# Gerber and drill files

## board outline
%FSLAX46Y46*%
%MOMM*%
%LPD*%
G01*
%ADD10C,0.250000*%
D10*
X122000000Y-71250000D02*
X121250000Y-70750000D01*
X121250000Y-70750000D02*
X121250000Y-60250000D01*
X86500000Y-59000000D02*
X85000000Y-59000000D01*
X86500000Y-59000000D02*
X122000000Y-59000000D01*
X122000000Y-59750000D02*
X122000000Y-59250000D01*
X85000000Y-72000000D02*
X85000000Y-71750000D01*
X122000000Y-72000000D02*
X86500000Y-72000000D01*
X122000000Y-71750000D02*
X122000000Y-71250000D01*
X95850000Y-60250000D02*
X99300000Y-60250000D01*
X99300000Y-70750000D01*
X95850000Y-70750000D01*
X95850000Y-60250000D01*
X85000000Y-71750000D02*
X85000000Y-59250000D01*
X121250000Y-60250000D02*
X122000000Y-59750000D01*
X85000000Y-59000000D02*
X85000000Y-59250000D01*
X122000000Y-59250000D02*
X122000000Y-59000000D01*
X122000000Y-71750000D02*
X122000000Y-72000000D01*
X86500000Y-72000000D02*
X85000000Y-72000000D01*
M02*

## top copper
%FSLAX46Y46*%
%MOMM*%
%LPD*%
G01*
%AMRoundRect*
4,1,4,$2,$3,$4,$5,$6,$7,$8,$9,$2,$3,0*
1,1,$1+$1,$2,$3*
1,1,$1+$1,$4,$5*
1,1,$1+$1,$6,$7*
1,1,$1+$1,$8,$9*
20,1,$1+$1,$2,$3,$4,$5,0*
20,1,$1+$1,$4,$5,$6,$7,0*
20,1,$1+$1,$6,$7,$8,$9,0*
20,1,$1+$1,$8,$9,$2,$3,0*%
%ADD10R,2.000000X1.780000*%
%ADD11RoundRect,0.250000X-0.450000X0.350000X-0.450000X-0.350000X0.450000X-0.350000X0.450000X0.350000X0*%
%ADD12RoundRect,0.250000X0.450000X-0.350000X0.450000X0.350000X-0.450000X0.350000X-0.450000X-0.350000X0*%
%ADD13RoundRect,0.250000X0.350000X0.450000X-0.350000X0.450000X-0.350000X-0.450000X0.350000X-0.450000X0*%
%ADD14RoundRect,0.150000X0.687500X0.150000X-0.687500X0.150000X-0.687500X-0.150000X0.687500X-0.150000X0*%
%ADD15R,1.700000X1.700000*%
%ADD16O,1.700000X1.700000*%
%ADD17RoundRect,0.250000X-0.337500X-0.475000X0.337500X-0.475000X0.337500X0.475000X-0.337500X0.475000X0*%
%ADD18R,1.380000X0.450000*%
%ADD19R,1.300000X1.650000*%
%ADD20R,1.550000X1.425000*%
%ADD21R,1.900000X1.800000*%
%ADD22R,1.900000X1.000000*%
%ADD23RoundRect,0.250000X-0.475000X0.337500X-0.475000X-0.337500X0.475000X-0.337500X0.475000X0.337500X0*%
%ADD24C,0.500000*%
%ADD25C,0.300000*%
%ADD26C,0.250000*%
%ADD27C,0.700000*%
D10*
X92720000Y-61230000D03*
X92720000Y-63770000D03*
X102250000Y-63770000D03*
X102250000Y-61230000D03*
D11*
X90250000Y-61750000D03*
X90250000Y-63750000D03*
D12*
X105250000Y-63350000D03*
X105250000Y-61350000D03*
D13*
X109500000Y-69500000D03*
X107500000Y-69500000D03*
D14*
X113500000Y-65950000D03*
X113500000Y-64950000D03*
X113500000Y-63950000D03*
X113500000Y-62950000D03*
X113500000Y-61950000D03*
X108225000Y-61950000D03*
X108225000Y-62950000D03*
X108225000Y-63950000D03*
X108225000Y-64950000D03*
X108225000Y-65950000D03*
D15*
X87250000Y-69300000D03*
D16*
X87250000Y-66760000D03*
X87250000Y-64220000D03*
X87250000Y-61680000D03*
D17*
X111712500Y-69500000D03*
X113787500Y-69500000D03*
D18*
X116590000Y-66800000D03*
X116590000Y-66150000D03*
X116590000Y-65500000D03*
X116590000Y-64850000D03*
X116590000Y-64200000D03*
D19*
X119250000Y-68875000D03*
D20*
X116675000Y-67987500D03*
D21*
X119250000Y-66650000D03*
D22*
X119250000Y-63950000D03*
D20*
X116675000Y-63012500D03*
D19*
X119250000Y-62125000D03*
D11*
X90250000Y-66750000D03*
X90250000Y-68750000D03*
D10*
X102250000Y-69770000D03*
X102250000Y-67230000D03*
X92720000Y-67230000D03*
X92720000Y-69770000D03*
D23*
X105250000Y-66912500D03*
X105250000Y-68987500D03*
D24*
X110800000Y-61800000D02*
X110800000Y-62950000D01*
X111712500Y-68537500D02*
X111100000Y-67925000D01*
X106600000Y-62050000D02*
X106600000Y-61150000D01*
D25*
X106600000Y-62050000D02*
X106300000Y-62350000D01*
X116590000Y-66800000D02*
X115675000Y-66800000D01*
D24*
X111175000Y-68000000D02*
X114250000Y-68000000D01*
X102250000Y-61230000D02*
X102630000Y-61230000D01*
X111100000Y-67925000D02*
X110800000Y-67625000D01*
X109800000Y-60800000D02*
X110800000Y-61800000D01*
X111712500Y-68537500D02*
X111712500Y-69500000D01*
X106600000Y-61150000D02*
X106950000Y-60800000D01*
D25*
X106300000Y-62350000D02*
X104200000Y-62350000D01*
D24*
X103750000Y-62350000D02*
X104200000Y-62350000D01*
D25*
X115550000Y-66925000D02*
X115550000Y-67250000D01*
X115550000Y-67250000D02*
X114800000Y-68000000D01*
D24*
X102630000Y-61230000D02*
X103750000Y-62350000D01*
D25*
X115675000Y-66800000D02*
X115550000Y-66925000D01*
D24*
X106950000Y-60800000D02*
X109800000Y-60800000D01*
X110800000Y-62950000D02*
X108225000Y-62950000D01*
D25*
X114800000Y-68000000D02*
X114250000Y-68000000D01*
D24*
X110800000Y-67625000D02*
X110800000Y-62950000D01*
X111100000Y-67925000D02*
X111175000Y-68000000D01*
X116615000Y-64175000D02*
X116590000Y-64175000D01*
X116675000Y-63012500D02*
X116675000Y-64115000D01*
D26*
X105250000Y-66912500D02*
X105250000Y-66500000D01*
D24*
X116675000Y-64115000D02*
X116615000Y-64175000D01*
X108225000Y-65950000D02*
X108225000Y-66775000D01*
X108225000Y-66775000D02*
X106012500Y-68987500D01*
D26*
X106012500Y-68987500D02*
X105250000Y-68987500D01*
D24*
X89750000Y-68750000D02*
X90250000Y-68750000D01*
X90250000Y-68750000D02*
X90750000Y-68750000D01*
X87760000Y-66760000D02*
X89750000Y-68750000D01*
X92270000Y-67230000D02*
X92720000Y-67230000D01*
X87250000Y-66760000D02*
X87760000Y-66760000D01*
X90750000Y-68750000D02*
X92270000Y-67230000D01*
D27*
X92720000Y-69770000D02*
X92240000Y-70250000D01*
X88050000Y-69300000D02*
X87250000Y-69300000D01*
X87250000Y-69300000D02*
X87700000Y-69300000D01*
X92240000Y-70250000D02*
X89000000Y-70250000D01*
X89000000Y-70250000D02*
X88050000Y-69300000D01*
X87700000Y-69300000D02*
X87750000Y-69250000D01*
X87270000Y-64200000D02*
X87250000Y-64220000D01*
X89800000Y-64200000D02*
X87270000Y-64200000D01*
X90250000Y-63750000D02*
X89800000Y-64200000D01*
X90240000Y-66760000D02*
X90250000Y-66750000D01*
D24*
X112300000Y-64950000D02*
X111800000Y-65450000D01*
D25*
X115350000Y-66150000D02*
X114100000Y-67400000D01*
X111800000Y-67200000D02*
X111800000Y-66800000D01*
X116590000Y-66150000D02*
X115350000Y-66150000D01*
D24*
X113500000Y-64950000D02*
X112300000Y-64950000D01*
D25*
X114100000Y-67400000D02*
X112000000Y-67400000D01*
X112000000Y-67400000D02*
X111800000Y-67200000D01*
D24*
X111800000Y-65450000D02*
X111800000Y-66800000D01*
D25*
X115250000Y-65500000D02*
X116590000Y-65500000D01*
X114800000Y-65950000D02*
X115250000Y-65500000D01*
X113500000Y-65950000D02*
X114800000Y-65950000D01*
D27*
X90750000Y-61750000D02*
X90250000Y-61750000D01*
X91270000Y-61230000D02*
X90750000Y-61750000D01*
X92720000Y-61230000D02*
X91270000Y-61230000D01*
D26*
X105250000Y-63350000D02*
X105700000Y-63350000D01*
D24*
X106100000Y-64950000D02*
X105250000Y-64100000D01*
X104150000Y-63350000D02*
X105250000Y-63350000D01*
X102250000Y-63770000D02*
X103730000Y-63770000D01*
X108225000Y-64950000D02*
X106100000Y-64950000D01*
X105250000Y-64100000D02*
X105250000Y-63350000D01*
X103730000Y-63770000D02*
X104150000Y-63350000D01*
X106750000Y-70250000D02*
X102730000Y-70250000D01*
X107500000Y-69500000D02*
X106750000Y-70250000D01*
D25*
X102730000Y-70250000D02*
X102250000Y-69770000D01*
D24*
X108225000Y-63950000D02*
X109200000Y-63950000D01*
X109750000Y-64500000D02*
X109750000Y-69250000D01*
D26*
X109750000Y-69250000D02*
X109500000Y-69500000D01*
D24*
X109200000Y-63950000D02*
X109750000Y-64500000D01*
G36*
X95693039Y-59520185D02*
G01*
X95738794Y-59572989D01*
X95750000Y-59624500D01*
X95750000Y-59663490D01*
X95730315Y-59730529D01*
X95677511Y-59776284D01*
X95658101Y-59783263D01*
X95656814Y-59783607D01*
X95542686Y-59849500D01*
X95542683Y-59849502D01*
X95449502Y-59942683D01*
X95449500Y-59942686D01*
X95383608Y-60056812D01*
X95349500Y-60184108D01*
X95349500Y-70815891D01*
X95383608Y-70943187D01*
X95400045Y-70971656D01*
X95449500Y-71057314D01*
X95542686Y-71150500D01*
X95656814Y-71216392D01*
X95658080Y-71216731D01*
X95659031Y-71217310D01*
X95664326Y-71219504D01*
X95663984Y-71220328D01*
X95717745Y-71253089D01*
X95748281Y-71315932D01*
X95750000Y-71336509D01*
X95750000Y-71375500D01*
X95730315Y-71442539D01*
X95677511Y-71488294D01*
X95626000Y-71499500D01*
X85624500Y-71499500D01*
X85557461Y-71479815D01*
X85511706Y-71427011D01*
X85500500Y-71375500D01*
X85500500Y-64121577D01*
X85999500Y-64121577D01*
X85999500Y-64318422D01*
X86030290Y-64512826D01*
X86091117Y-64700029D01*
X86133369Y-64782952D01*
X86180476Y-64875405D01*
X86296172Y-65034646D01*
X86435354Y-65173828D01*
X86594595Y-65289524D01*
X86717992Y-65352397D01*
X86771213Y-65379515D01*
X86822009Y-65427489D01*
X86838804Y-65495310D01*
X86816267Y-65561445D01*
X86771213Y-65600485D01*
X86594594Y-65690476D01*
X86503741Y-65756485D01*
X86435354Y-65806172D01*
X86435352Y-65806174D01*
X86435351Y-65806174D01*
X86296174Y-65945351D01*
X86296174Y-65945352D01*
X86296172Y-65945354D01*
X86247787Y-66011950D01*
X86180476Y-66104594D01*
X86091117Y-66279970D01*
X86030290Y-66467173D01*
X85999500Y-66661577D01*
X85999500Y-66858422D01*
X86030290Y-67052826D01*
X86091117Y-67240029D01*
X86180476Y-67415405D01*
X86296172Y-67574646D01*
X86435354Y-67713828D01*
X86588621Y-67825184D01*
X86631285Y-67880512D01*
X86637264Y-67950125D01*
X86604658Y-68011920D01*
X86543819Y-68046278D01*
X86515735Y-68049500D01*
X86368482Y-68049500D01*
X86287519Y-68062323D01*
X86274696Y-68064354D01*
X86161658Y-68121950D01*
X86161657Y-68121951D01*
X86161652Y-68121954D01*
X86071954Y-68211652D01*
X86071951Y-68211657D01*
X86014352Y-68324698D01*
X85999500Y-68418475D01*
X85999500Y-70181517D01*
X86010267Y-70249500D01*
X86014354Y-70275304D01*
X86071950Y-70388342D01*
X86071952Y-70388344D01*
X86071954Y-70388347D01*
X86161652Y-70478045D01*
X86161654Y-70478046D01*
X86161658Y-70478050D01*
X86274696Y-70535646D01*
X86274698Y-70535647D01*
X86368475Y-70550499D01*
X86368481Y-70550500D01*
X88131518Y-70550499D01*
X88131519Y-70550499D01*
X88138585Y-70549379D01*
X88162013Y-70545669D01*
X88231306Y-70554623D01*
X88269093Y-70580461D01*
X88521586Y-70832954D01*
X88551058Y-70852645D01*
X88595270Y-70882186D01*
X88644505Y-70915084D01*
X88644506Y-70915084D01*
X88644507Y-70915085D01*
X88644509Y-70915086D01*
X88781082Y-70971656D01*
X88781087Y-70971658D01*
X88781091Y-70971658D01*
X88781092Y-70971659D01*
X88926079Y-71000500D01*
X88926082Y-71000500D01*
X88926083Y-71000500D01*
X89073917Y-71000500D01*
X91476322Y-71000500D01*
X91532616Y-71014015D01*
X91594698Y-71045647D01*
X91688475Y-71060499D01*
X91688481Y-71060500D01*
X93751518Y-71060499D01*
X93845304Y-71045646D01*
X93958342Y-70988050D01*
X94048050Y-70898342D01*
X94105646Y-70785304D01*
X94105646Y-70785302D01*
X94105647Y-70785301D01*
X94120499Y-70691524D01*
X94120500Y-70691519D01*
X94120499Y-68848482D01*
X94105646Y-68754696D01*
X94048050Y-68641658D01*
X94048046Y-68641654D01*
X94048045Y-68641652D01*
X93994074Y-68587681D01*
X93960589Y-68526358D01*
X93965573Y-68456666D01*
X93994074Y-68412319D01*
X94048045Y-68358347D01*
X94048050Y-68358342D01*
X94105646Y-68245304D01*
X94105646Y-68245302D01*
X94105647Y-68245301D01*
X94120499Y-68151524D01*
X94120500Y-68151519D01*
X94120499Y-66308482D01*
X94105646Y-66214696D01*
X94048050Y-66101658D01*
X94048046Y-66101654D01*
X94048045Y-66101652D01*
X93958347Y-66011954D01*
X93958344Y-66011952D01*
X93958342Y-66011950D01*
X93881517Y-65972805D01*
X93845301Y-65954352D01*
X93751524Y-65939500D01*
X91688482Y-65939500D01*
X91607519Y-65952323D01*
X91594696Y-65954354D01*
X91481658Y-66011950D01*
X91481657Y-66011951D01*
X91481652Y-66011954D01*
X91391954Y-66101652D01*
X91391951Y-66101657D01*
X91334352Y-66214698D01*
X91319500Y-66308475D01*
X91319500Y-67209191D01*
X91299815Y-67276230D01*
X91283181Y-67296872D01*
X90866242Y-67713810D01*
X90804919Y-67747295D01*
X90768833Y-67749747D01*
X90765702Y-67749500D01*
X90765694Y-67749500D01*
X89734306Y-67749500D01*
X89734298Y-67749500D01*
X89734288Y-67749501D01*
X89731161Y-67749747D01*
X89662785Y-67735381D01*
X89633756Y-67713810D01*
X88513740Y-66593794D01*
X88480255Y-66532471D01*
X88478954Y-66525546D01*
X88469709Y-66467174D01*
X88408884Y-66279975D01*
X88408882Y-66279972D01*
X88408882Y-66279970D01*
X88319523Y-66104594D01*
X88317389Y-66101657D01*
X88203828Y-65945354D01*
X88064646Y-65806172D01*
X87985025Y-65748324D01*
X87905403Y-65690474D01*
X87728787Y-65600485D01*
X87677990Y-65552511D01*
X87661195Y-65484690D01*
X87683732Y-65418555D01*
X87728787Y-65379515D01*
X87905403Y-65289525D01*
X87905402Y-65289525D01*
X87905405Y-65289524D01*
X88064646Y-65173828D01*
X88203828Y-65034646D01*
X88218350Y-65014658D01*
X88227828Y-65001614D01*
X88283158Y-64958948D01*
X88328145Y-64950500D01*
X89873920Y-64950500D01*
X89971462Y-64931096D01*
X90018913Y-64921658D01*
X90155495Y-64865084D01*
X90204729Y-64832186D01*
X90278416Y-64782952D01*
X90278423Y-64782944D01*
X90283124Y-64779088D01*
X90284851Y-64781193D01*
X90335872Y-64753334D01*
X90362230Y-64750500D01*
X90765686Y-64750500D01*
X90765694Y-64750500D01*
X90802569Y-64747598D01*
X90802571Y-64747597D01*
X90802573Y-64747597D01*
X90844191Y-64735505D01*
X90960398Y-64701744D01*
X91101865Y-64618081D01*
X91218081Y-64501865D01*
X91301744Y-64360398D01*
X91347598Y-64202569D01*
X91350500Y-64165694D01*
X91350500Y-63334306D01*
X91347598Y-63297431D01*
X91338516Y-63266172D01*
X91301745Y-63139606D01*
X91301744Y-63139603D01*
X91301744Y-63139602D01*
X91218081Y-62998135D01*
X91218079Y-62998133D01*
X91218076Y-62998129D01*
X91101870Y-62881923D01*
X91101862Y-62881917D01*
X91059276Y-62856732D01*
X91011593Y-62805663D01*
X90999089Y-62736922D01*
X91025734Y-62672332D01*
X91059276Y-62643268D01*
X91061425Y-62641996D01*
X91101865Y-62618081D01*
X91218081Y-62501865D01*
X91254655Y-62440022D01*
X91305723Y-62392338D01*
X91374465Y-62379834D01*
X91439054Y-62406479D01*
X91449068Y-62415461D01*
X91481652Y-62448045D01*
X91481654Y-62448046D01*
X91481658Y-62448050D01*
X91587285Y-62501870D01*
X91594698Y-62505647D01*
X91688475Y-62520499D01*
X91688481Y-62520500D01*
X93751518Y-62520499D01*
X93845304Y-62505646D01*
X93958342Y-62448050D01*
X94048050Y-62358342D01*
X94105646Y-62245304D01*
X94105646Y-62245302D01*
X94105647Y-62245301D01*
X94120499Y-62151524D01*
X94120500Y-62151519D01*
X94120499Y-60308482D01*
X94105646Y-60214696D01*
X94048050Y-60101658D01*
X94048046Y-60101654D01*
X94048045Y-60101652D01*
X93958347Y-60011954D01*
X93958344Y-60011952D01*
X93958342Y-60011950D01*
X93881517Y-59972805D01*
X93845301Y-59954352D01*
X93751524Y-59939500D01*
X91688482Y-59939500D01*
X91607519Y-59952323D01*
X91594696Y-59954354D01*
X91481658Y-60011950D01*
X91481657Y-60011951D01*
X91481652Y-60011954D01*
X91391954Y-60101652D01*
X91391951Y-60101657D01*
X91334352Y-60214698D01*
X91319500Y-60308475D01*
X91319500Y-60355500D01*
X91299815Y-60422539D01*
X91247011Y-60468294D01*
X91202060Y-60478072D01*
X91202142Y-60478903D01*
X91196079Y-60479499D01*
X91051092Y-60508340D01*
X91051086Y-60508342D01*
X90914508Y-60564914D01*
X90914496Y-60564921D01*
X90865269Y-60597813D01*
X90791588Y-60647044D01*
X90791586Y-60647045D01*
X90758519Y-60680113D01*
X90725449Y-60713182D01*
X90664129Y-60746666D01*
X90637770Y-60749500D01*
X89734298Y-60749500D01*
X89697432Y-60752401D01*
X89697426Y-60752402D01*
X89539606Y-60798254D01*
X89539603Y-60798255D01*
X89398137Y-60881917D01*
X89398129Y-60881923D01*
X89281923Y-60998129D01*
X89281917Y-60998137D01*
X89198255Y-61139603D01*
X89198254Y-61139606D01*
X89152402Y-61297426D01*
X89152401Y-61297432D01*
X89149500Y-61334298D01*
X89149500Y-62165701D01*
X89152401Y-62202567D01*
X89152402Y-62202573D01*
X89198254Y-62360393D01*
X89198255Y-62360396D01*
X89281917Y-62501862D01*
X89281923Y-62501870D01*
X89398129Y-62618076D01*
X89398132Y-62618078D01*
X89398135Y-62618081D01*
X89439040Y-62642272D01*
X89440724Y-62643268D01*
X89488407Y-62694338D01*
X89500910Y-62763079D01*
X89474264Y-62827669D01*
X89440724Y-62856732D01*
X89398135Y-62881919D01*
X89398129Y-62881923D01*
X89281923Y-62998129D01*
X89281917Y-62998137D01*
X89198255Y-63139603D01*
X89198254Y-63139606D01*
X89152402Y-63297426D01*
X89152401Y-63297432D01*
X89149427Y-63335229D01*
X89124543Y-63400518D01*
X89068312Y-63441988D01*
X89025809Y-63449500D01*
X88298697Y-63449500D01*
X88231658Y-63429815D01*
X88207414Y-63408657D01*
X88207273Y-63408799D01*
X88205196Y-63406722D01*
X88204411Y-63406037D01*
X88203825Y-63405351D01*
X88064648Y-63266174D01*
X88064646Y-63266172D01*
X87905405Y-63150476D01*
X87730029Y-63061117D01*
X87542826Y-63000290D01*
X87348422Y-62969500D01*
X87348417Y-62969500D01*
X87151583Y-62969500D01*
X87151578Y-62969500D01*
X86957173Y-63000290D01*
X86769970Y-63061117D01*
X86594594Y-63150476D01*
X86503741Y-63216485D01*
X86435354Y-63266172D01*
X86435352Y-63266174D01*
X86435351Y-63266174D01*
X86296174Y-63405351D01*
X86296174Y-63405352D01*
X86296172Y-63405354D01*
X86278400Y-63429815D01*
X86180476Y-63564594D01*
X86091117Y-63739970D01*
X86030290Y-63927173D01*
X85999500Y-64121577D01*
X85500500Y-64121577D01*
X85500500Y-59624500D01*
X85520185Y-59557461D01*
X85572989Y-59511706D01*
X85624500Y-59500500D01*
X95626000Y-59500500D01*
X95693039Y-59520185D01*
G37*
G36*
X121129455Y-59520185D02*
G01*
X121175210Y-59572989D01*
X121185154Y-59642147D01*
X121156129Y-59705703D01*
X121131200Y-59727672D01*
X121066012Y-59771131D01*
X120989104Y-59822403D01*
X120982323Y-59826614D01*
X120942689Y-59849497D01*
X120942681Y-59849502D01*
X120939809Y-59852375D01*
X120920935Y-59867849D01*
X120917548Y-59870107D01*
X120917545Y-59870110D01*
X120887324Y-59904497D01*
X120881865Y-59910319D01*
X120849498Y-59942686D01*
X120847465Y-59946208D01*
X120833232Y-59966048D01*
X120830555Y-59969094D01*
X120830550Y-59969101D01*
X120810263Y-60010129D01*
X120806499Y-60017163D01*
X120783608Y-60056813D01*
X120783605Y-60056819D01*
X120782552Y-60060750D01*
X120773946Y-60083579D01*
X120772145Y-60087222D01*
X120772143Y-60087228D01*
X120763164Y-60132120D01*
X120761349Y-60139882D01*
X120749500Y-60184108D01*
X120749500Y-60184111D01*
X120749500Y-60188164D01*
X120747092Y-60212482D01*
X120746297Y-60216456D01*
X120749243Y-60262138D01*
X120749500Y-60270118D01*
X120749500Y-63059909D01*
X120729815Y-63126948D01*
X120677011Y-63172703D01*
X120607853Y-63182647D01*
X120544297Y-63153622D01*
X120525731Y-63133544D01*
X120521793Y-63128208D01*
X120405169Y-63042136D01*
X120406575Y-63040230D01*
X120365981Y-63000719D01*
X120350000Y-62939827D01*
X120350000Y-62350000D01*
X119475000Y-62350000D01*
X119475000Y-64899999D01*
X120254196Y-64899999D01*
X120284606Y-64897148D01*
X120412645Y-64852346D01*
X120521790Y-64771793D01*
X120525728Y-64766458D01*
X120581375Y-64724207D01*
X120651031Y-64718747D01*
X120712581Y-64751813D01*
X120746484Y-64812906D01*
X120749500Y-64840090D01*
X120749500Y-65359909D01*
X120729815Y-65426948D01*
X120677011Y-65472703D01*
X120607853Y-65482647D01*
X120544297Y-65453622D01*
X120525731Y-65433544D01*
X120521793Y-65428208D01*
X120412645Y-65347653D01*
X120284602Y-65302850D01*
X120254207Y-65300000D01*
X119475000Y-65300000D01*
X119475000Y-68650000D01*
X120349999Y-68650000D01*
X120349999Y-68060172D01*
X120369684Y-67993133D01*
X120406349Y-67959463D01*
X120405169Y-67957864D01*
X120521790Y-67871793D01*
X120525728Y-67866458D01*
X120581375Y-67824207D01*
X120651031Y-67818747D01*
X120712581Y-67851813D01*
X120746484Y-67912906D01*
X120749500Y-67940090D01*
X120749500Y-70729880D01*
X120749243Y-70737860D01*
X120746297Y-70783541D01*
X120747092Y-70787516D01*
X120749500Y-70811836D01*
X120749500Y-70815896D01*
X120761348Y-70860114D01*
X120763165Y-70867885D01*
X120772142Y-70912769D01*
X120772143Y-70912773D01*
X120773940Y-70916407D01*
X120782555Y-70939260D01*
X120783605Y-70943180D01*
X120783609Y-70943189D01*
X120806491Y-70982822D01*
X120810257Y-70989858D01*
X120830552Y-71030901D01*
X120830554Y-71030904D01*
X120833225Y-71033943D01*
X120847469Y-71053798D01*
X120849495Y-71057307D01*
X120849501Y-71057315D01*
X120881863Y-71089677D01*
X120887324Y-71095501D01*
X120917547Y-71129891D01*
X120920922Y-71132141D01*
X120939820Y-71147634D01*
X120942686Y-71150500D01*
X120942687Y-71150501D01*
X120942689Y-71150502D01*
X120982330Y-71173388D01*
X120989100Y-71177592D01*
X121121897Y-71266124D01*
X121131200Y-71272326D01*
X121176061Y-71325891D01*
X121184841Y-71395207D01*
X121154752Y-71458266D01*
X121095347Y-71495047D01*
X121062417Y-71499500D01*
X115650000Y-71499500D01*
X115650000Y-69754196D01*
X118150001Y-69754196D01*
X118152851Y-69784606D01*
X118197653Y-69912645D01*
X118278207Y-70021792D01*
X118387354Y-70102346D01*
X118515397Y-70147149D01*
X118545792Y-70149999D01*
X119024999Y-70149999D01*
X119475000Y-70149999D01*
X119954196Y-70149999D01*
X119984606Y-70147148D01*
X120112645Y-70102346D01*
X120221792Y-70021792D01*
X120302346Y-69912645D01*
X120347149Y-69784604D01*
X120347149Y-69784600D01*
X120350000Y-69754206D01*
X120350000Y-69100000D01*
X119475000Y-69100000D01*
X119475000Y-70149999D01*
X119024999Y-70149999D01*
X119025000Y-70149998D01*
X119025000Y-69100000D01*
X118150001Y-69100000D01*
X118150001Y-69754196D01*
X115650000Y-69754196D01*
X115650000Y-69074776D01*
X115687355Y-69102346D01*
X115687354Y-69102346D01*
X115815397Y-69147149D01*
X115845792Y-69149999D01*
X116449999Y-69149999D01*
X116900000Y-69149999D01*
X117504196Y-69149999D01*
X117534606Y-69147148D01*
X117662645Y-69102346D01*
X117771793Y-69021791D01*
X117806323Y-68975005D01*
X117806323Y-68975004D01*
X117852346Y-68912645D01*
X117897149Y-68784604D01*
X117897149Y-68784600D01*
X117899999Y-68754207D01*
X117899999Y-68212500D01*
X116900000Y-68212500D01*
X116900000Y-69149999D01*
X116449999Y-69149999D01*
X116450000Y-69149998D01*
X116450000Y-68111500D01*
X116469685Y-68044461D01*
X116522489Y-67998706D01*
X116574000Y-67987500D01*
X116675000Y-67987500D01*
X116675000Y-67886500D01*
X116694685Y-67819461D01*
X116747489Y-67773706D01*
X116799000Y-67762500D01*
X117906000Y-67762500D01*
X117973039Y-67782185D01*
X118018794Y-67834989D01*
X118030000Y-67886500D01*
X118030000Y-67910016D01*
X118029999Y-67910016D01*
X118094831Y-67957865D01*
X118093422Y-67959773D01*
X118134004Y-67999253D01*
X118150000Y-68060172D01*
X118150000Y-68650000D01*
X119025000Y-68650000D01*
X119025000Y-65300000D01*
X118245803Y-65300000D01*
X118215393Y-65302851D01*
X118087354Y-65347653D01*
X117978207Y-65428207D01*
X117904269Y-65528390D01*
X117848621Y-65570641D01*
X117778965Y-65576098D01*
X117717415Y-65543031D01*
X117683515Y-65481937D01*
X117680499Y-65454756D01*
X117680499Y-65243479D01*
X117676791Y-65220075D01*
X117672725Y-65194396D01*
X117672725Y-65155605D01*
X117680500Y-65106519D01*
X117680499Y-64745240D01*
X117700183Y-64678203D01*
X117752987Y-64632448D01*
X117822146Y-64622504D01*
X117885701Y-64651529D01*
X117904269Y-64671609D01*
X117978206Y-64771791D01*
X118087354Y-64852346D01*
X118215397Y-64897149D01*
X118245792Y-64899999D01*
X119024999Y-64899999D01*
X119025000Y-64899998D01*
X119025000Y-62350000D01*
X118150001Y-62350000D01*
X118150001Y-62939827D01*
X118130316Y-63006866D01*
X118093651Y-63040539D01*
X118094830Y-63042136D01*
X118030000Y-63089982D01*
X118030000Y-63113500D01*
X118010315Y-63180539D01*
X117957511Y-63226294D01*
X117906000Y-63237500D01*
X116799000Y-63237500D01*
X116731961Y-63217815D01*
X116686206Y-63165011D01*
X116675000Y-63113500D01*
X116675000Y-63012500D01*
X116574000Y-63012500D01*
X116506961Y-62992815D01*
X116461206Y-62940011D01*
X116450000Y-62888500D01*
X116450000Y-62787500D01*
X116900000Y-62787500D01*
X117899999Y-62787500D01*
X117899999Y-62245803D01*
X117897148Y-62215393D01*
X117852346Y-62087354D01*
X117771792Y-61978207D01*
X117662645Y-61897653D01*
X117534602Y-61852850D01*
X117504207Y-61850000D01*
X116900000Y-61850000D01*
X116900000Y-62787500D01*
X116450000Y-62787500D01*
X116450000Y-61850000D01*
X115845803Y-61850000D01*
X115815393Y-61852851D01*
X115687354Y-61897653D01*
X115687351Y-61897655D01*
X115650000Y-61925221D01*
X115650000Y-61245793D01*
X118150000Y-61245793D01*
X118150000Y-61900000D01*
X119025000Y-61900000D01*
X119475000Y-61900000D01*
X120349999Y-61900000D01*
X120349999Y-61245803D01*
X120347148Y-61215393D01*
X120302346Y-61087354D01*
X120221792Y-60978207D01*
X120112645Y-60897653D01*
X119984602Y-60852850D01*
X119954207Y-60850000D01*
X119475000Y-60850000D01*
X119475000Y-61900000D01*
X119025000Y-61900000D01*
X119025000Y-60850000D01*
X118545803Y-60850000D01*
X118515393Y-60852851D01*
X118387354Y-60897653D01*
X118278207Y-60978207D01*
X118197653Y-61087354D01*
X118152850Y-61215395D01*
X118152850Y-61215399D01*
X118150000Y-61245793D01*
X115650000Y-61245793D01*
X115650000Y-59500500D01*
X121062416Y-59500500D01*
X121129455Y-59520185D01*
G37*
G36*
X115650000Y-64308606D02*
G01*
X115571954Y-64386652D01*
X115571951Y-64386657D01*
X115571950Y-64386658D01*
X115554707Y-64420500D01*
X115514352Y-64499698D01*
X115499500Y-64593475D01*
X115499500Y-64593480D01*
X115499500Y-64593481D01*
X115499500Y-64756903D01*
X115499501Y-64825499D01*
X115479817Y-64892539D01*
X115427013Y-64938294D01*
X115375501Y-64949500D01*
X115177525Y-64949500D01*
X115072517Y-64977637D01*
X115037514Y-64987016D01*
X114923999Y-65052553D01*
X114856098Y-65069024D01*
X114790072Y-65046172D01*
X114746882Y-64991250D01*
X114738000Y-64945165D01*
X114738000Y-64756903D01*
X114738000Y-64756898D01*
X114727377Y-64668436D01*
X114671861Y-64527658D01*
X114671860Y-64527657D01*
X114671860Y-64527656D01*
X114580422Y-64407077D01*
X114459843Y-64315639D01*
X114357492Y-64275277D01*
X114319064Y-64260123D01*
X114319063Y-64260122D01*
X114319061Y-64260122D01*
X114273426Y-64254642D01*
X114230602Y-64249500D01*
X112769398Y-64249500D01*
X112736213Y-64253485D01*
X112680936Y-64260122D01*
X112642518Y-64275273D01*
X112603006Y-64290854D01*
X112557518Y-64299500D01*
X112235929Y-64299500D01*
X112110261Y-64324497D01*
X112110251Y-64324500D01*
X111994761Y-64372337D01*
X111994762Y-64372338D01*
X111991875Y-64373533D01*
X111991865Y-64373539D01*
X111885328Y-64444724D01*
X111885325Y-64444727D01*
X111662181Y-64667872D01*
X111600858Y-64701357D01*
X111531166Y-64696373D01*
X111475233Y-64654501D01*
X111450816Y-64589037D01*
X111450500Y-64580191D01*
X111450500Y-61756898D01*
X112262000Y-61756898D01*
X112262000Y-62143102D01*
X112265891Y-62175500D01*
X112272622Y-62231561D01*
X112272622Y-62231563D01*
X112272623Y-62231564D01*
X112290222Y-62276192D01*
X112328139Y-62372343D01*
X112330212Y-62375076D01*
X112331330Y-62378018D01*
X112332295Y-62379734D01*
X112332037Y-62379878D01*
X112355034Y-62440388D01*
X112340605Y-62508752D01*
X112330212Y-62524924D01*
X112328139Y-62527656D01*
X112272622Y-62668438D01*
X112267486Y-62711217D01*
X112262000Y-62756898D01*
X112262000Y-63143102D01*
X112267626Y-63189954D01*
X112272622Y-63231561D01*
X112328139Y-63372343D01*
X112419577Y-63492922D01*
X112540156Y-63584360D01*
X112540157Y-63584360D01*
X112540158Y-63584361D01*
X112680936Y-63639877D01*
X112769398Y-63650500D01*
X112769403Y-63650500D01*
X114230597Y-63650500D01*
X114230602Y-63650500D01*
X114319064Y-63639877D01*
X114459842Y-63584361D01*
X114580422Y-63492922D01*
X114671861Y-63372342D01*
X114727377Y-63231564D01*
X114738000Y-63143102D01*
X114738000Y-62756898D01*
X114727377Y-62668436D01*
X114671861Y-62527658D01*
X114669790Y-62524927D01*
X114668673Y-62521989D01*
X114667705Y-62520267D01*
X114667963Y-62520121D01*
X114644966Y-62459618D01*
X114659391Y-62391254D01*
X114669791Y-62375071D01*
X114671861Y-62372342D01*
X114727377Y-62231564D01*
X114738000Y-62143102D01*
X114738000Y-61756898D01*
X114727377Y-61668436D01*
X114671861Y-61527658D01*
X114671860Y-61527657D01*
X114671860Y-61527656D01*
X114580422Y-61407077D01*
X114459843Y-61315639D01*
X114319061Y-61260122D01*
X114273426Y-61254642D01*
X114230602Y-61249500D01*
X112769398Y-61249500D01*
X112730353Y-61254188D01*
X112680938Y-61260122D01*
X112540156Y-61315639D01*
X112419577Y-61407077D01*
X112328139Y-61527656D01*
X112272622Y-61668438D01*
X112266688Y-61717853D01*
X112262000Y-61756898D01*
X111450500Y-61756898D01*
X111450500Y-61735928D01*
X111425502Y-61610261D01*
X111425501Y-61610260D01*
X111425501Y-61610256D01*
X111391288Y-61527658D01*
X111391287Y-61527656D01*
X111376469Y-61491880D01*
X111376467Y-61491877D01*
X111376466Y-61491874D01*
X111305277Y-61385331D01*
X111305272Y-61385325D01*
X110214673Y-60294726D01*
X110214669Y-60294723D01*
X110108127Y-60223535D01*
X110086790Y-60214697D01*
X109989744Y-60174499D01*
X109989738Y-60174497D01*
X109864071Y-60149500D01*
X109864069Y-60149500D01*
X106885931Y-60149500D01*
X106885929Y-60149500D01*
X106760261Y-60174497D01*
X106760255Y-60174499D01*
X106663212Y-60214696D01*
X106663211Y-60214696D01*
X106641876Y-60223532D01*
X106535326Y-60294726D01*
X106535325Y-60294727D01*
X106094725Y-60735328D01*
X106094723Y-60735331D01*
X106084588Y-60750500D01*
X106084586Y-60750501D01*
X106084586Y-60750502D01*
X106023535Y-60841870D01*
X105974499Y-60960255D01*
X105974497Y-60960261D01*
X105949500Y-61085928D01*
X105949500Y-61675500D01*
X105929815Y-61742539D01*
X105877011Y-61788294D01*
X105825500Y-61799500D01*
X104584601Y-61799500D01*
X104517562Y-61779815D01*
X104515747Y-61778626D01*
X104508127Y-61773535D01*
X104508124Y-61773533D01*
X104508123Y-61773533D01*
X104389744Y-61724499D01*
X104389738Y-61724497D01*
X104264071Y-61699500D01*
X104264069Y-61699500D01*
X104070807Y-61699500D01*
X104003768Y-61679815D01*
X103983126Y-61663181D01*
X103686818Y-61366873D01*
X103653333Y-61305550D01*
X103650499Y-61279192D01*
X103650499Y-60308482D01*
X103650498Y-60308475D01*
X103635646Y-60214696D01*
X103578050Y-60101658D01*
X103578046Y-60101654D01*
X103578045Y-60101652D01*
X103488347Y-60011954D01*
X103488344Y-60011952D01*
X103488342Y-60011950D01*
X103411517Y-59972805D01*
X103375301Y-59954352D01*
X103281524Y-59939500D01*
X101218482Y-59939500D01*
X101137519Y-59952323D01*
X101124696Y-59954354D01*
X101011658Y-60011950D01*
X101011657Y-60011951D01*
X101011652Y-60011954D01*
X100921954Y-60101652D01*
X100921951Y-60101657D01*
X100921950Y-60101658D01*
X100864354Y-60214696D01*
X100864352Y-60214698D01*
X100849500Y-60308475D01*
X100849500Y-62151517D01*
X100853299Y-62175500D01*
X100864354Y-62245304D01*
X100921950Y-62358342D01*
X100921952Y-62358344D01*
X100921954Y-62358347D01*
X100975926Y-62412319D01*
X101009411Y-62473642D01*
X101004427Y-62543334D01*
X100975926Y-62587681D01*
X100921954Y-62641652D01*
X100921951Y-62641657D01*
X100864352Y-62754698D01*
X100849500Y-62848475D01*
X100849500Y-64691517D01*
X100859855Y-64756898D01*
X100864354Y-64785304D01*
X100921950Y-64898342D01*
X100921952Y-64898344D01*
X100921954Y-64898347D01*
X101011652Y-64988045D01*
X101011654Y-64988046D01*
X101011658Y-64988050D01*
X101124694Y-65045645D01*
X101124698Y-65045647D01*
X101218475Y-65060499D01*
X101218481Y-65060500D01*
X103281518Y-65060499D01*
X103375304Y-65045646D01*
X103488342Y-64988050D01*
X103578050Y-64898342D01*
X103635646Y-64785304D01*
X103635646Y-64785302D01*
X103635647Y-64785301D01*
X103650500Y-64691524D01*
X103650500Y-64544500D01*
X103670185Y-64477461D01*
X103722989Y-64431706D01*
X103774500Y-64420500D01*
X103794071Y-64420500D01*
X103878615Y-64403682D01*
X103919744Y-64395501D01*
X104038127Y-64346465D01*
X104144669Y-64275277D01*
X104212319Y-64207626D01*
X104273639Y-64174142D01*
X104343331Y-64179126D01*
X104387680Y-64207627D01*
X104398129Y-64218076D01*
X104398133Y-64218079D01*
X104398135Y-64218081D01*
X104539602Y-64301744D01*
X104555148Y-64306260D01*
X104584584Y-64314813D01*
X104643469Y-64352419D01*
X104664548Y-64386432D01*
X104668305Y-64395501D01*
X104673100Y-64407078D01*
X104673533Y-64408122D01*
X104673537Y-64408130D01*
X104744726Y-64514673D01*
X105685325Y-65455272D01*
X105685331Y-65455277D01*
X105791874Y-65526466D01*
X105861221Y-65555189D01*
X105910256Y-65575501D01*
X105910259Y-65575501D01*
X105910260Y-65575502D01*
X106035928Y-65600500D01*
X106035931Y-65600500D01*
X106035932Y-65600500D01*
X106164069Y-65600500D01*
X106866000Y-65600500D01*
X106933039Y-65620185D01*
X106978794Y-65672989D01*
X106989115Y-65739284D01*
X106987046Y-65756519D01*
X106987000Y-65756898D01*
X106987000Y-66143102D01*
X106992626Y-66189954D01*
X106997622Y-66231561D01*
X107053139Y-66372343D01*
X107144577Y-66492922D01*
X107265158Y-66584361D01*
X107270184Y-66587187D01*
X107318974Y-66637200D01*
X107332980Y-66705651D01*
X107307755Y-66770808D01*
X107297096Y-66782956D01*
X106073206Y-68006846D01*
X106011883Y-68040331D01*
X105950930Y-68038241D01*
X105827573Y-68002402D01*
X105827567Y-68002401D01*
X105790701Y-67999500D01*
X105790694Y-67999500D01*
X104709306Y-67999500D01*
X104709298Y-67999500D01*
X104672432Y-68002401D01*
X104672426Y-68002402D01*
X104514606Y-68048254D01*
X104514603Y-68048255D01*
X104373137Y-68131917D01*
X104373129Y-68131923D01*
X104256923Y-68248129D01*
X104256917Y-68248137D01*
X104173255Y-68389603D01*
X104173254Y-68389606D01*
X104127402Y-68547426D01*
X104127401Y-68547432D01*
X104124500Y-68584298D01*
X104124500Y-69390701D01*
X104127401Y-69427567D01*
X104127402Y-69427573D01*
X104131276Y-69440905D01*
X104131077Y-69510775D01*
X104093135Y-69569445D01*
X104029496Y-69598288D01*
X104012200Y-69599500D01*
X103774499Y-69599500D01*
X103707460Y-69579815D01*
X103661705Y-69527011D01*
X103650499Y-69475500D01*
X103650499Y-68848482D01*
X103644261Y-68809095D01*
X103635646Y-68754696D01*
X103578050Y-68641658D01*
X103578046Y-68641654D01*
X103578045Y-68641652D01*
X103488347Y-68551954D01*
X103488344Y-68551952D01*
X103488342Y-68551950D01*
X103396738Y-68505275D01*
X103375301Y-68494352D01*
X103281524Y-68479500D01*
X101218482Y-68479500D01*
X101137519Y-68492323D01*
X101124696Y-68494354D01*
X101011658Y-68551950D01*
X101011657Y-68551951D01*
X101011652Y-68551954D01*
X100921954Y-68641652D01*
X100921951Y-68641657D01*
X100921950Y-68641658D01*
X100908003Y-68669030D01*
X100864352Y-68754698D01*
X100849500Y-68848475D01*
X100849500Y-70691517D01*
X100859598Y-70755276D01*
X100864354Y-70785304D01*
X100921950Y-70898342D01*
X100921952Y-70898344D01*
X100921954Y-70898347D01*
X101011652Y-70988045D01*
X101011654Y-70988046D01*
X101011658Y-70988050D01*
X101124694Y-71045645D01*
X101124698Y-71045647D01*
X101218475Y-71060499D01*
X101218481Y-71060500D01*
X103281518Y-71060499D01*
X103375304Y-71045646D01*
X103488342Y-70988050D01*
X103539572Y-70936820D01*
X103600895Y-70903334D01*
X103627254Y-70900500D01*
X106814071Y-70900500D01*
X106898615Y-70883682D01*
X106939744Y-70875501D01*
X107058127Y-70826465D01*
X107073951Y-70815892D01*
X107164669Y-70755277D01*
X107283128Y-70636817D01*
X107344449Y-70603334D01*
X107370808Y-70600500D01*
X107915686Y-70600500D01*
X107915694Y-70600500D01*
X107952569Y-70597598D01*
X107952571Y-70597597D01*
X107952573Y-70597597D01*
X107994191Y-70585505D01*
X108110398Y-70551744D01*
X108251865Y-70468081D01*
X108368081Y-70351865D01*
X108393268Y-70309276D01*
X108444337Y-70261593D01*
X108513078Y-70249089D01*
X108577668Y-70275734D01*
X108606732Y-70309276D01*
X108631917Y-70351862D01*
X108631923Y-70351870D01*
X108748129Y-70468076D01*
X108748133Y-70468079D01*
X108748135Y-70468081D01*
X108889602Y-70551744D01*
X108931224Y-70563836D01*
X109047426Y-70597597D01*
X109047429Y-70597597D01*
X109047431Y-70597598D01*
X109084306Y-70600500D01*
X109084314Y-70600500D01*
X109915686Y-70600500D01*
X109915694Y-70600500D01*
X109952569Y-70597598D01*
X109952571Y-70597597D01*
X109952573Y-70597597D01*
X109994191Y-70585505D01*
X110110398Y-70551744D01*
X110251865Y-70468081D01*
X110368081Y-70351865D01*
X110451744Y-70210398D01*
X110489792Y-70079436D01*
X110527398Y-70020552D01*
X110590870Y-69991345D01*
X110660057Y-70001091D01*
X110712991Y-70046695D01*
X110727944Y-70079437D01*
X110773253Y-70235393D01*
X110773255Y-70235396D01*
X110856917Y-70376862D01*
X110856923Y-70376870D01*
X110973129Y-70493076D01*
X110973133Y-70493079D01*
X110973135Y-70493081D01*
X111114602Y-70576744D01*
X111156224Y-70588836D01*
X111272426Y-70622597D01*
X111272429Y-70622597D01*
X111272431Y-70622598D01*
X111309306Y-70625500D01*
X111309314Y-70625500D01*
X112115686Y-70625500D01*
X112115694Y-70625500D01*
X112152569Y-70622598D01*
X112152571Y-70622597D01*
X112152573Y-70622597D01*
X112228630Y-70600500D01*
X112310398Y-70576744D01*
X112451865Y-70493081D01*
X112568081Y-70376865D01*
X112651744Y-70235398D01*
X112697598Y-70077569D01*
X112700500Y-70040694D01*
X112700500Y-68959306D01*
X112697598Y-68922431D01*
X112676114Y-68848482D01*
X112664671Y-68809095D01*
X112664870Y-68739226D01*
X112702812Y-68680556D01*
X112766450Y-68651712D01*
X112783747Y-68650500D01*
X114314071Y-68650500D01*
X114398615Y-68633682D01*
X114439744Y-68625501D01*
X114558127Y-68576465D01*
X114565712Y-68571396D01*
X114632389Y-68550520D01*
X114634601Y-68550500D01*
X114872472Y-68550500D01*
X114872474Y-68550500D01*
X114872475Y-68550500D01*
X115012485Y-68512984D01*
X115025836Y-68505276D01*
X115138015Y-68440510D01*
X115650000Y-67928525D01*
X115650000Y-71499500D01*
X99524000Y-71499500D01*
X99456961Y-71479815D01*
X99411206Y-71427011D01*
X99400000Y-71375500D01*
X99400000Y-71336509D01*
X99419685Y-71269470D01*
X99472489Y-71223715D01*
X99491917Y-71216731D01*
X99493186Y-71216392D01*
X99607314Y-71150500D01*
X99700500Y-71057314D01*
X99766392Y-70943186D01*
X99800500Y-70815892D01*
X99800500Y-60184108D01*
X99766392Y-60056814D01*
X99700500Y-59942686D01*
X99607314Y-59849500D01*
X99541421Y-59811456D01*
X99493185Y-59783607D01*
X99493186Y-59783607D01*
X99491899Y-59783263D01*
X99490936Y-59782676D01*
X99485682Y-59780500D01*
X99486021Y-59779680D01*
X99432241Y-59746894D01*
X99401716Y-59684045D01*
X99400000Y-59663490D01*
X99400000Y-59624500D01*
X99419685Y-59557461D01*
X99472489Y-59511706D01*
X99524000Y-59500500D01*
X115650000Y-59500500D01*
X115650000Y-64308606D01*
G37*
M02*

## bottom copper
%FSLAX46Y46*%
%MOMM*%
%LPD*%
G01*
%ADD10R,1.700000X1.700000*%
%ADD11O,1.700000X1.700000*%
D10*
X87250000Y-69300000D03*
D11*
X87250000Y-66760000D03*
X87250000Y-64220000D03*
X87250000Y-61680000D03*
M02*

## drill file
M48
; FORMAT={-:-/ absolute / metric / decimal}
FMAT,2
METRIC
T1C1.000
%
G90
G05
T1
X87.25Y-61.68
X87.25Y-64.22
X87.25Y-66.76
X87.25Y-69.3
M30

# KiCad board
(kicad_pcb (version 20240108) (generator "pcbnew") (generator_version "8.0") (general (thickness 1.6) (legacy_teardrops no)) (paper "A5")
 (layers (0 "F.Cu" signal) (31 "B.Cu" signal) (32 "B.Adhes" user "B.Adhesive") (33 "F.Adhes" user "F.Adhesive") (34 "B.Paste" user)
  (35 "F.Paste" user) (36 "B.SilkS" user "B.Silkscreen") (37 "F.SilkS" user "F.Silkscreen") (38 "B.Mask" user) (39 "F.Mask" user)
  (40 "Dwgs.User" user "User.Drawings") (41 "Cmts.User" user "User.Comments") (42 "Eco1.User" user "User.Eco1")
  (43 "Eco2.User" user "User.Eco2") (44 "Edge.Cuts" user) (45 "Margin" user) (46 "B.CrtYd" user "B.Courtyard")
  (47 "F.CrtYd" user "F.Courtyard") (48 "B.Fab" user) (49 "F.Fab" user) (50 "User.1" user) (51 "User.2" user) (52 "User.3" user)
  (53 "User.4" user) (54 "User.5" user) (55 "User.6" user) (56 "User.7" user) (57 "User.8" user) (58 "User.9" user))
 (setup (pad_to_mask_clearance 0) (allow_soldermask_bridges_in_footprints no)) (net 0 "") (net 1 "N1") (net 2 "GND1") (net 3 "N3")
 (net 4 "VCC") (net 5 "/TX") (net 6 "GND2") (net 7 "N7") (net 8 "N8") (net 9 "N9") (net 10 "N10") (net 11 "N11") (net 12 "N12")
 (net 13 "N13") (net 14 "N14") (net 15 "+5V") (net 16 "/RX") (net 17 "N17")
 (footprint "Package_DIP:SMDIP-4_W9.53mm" (layer "F.Cu") (at 97.485 62.5)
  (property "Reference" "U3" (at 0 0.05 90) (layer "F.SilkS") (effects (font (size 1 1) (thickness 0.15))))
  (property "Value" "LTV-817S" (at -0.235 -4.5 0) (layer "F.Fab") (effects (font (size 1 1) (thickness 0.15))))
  (pad "1" smd rect (at -4.765 -1.27) (size 2 1.78) (layers "F.Cu" "F.Paste" "F.Mask") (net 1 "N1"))
  (pad "2" smd rect (at -4.765 1.27) (size 2 1.78) (layers "F.Cu" "F.Paste" "F.Mask") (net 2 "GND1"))
  (pad "3" smd rect (at 4.765 1.27) (size 2 1.78) (layers "F.Cu" "F.Paste" "F.Mask") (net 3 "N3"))
  (pad "4" smd rect (at 4.765 -1.27) (size 2 1.78) (layers "F.Cu" "F.Paste" "F.Mask") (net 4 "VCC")))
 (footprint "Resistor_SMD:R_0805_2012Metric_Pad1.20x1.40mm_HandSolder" (layer "F.Cu") (at 90.25 62.75 -90)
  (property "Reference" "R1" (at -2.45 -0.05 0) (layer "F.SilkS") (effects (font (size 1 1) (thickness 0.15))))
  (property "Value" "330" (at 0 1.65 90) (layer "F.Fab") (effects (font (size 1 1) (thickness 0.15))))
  (pad "1" smd roundrect (at -1 0 270) (size 1.2 1.4) (layers "F.Cu" "F.Paste" "F.Mask") (roundrect_rratio 0.208333) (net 1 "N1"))
  (pad "2" smd roundrect (at 1 0 270) (size 1.2 1.4) (layers "F.Cu" "F.Paste" "F.Mask") (roundrect_rratio 0.208333) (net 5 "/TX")))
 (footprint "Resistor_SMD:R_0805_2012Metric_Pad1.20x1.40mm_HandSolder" (layer "F.Cu") (at 105.25 62.35 90)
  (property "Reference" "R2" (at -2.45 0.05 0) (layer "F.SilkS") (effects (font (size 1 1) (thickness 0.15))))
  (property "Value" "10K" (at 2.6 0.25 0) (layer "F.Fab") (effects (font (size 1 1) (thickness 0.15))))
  (pad "1" smd roundrect (at -1 0 90) (size 1.2 1.4) (layers "F.Cu" "F.Paste" "F.Mask") (roundrect_rratio 0.208333) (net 3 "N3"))
  (pad "2" smd roundrect (at 1 0 90) (size 1.2 1.4) (layers "F.Cu" "F.Paste" "F.Mask") (roundrect_rratio 0.208333) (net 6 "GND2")))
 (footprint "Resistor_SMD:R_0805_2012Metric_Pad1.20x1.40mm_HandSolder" (layer "F.Cu") (at 108.5 69.5 180)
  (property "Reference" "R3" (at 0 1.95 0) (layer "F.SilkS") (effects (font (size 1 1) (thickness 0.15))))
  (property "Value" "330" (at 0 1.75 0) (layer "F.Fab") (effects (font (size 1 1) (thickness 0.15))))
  (pad "1" smd roundrect (at -1 0 180) (size 1.2 1.4) (layers "F.Cu" "F.Paste" "F.Mask") (roundrect_rratio 0.208333) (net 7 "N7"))
  (pad "2" smd roundrect (at 1 0 180) (size 1.2 1.4) (layers "F.Cu" "F.Paste" "F.Mask") (roundrect_rratio 0.208333) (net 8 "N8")))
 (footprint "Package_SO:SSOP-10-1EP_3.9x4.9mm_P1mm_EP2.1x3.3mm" (layer "F.Cu") (at 110.8625 63.95 180)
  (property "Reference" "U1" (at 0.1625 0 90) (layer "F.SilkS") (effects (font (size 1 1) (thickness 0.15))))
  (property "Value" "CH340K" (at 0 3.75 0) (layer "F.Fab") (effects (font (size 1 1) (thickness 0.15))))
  (pad "1" smd roundrect (at -2.6375 -2 180) (size 1.675 0.6) (layers "F.Cu" "F.Paste" "F.Mask") (roundrect_rratio 0.25) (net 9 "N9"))
  (pad "2" smd roundrect (at -2.6375 -1 180) (size 1.675 0.6) (layers "F.Cu" "F.Paste" "F.Mask") (roundrect_rratio 0.25) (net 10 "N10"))
  (pad "3" smd roundrect (at -2.6375 0 180) (size 1.675 0.6) (layers "F.Cu" "F.Paste" "F.Mask") (roundrect_rratio 0.25) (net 6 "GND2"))
  (pad "4" smd roundrect (at -2.6375 1 180) (size 1.675 0.6) (layers "F.Cu" "F.Paste" "F.Mask") (roundrect_rratio 0.25) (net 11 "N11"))
  (pad "5" smd roundrect (at -2.6375 2 180) (size 1.675 0.6) (layers "F.Cu" "F.Paste" "F.Mask") (roundrect_rratio 0.25) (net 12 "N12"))
  (pad "6" smd roundrect (at 2.6375 2 180) (size 1.675 0.6) (layers "F.Cu" "F.Paste" "F.Mask") (roundrect_rratio 0.25) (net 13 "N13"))
  (pad "7" smd roundrect (at 2.6375 1 180) (size 1.675 0.6) (layers "F.Cu" "F.Paste" "F.Mask") (roundrect_rratio 0.25) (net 4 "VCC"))
  (pad "8" smd roundrect (at 2.6375 0 180) (size 1.675 0.6) (layers "F.Cu" "F.Paste" "F.Mask") (roundrect_rratio 0.25) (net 7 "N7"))
  (pad "9" smd roundrect (at 2.6375 -1 180) (size 1.675 0.6) (layers "F.Cu" "F.Paste" "F.Mask") (roundrect_rratio 0.25) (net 3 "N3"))
  (pad "10" smd roundrect (at 2.6375 -2 180) (size 1.675 0.6) (layers "F.Cu" "F.Paste" "F.Mask") (roundrect_rratio 0.25) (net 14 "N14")))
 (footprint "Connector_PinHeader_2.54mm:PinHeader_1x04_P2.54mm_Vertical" (layer "F.Cu") (at 87.25 69.3 180)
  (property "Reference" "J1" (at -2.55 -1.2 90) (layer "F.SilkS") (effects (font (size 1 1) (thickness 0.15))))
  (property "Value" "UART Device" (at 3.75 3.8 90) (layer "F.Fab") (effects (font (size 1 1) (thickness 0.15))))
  (pad "1" thru_hole rect (at 0 0 180) (size 1.7 1.7) (drill 1) (layers "*.Cu" "*.Mask") (remove_unused_layers no) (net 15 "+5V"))
  (pad "2" thru_hole oval (at 0 2.54 180) (size 1.7 1.7) (drill 1) (layers "*.Cu" "*.Mask") (remove_unused_layers no) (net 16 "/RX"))
  (pad "3" thru_hole oval (at 0 5.08 180) (size 1.7 1.7) (drill 1) (layers "*.Cu" "*.Mask") (remove_unused_layers no) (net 5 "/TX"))
  (pad "4" thru_hole oval (at 0 7.62 180) (size 1.7 1.7) (drill 1) (layers "*.Cu" "*.Mask") (remove_unused_layers no) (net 2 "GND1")))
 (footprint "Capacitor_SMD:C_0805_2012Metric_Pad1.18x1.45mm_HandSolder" (layer "F.Cu") (at 112.75 69.5)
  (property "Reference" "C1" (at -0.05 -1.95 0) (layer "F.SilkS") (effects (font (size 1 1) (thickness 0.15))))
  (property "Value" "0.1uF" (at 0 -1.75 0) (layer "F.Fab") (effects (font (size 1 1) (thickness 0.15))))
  (pad "1" smd roundrect (at -1.0375 0) (size 1.175 1.45) (layers "F.Cu" "F.Paste" "F.Mask") (roundrect_rratio 0.212766) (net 4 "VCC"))
  (pad "2" smd roundrect (at 1.0375 0) (size 1.175 1.45) (layers "F.Cu" "F.Paste" "F.Mask") (roundrect_rratio 0.212766) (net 6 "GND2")))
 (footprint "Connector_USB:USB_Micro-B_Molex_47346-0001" (layer "F.Cu") (at 118.05 65.5 90)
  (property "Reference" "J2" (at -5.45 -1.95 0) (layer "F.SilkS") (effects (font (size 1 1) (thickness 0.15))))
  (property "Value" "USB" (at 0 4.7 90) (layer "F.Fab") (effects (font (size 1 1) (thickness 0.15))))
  (pad "1" smd rect (at -1.3 -1.46 90) (size 0.45 1.38) (layers "F.Cu" "F.Paste" "F.Mask") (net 4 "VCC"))
  (pad "2" smd rect (at -0.65 -1.46 90) (size 0.45 1.38) (layers "F.Cu" "F.Paste" "F.Mask") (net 10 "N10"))
  (pad "3" smd rect (at 0 -1.46 90) (size 0.45 1.38) (layers "F.Cu" "F.Paste" "F.Mask") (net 9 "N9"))
  (pad "4" smd rect (at 0.65 -1.46 90) (size 0.45 1.38) (layers "F.Cu" "F.Paste" "F.Mask") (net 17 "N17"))
  (pad "5" smd rect (at 1.3 -1.46 90) (size 0.45 1.38) (layers "F.Cu" "F.Paste" "F.Mask") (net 6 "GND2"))
  (pad "6" smd rect (at -3.375 1.2 90) (size 1.65 1.3) (layers "F.Cu" "F.Paste" "F.Mask") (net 6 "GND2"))
  (pad "6" smd rect (at -2.4875 -1.375 90) (size 1.425 1.55) (layers "F.Cu" "F.Paste" "F.Mask") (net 6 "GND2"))
  (pad "6" smd rect (at -1.15 1.2 90) (size 1.8 1.9) (layers "F.Cu" "F.Paste" "F.Mask") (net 6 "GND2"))
  (pad "6" smd rect (at 1.55 1.2 90) (size 1 1.9) (layers "F.Cu" "F.Paste" "F.Mask") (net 6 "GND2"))
  (pad "6" smd rect (at 2.4875 -1.375 90) (size 1.425 1.55) (layers "F.Cu" "F.Paste" "F.Mask") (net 6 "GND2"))
  (pad "6" smd rect (at 3.375 1.2 90) (size 1.65 1.3) (layers "F.Cu" "F.Paste" "F.Mask") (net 6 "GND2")))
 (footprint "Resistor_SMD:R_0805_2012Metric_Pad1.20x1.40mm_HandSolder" (layer "F.Cu") (at 90.25 67.75 -90)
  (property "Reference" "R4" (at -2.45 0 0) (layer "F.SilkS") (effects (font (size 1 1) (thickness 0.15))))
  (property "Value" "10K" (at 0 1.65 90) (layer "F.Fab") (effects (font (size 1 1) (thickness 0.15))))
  (pad "1" smd roundrect (at -1 0 270) (size 1.2 1.4) (layers "F.Cu" "F.Paste" "F.Mask") (roundrect_rratio 0.208333) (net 2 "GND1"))
  (pad "2" smd roundrect (at 1 0 270) (size 1.2 1.4) (layers "F.Cu" "F.Paste" "F.Mask") (roundrect_rratio 0.208333) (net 16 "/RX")))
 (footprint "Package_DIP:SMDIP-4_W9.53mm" (layer "F.Cu") (at 97.485 68.5 180)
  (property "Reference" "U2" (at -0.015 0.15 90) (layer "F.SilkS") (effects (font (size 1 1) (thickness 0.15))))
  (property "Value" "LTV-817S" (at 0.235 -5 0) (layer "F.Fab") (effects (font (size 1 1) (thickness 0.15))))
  (pad "1" smd rect (at -4.765 -1.27 180) (size 2 1.78) (layers "F.Cu" "F.Paste" "F.Mask") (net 8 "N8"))
  (pad "2" smd rect (at -4.765 1.27 180) (size 2 1.78) (layers "F.Cu" "F.Paste" "F.Mask") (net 6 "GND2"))
  (pad "3" smd rect (at 4.765 1.27 180) (size 2 1.78) (layers "F.Cu" "F.Paste" "F.Mask") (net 16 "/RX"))
  (pad "4" smd rect (at 4.765 -1.27 180) (size 2 1.78) (layers "F.Cu" "F.Paste" "F.Mask") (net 15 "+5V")))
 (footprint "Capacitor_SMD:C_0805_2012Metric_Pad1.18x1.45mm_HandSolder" (layer "F.Cu") (at 105.25 67.95 -90)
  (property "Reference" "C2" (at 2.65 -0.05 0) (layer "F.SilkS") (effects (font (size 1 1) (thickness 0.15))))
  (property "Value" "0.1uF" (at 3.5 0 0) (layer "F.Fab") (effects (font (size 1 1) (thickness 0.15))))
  (pad "1" smd roundrect (at -1.0375 0 270) (size 1.175 1.45) (layers "F.Cu" "F.Paste" "F.Mask") (roundrect_rratio 0.212766) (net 6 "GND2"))
  (pad "2" smd roundrect (at 1.0375 0 270) (size 1.175 1.45) (layers "F.Cu" "F.Paste" "F.Mask") (roundrect_rratio 0.212766) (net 14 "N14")))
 (gr_line (start 122 71.25) (end 121.25 70.75) (stroke (width 0.25) (type default)) (layer "Edge.Cuts"))
 (gr_line (start 121.25 70.75) (end 121.25 60.25) (stroke (width 0.25) (type default)) (layer "Edge.Cuts"))
 (gr_line (start 86.5 59) (end 85 59) (stroke (width 0.25) (type default)) (layer "Edge.Cuts"))
 (gr_line (start 86.5 59) (end 122 59) (stroke (width 0.25) (type default)) (layer "Edge.Cuts"))
 (gr_line (start 122 59.75) (end 122 59.25) (stroke (width 0.25) (type default)) (layer "Edge.Cuts"))
 (gr_line (start 85 72) (end 85 71.75) (stroke (width 0.25) (type default)) (layer "Edge.Cuts"))
 (gr_line (start 122 72) (end 86.5 72) (stroke (width 0.25) (type default)) (layer "Edge.Cuts"))
 (gr_line (start 122 71.75) (end 122 71.25) (stroke (width 0.25) (type default)) (layer "Edge.Cuts"))
 (gr_rect (start 95.85 60.25) (end 99.3 70.75) (stroke (width 0.25) (type default)) (fill none) (layer "Edge.Cuts"))
 (gr_line (start 85 71.75) (end 85 59.25) (stroke (width 0.25) (type default)) (layer "Edge.Cuts"))
 (gr_line (start 121.25 60.25) (end 122 59.75) (stroke (width 0.25) (type default)) (layer "Edge.Cuts"))
 (gr_line (start 85 59) (end 85 59.25) (stroke (width 0.25) (type default)) (layer "Edge.Cuts"))
 (gr_line (start 122 59.25) (end 122 59) (stroke (width 0.25) (type default)) (layer "Edge.Cuts"))
 (gr_line (start 122 71.75) (end 122 72) (stroke (width 0.25) (type default)) (layer "Edge.Cuts"))
 (gr_line (start 86.5 72) (end 85 72) (stroke (width 0.25) (type default)) (layer "Edge.Cuts"))
 (segment (start 110.8 61.8) (end 110.8 62.95) (width 0.5) (layer "F.Cu") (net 4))
 (segment (start 111.7125 68.5375) (end 111.1 67.925) (width 0.5) (layer "F.Cu") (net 4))
 (segment (start 106.6 62.05) (end 106.6 61.15) (width 0.5) (layer "F.Cu") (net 4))
 (segment (start 106.6 62.05) (end 106.3 62.35) (width 0.3) (layer "F.Cu") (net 4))
 (segment (start 116.59 66.8) (end 115.675 66.8) (width 0.3) (layer "F.Cu") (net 4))
 (segment (start 111.175 68) (end 114.25 68) (width 0.5) (layer "F.Cu") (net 4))
 (segment (start 102.25 61.23) (end 102.63 61.23) (width 0.5) (layer "F.Cu") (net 4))
 (segment (start 111.1 67.925) (end 110.8 67.625) (width 0.5) (layer "F.Cu") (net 4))
 (segment (start 109.8 60.8) (end 110.8 61.8) (width 0.5) (layer "F.Cu") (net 4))
 (segment (start 111.7125 68.5375) (end 111.7125 69.5) (width 0.5) (layer "F.Cu") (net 4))
 (segment (start 106.6 61.15) (end 106.95 60.8) (width 0.5) (layer "F.Cu") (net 4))
 (segment (start 106.3 62.35) (end 104.2 62.35) (width 0.3) (layer "F.Cu") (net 4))
 (segment (start 103.75 62.35) (end 104.2 62.35) (width 0.5) (layer "F.Cu") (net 4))
 (segment (start 115.55 66.925) (end 115.55 67.25) (width 0.3) (layer "F.Cu") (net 4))
 (segment (start 115.55 67.25) (end 114.8 68) (width 0.3) (layer "F.Cu") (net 4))
 (segment (start 102.63 61.23) (end 103.75 62.35) (width 0.5) (layer "F.Cu") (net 4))
 (segment (start 115.675 66.8) (end 115.55 66.925) (width 0.3) (layer "F.Cu") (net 4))
 (segment (start 106.95 60.8) (end 109.8 60.8) (width 0.5) (layer "F.Cu") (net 4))
 (segment (start 110.8 62.95) (end 108.225 62.95) (width 0.5) (layer "F.Cu") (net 4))
 (segment (start 114.8 68) (end 114.25 68) (width 0.3) (layer "F.Cu") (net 4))
 (segment (start 110.8 67.625) (end 110.8 62.95) (width 0.5) (layer "F.Cu") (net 4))
 (segment (start 111.1 67.925) (end 111.175 68) (width 0.5) (layer "F.Cu") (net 4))
 (segment (start 116.615 64.175) (end 116.59 64.175) (width 0.5) (layer "F.Cu") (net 6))
 (segment (start 116.675 63.0125) (end 116.675 64.115) (width 0.5) (layer "F.Cu") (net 6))
 (segment (start 105.25 66.9125) (end 105.25 66.5) (width 0.25) (layer "F.Cu") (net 6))
 (segment (start 116.675 64.115) (end 116.615 64.175) (width 0.5) (layer "F.Cu") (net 6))
 (segment (start 108.225 65.95) (end 108.225 66.775) (width 0.5) (layer "F.Cu") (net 14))
 (segment (start 108.225 66.775) (end 106.0125 68.9875) (width 0.5) (layer "F.Cu") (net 14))
 (segment (start 106.0125 68.9875) (end 105.25 68.9875) (width 0.25) (layer "F.Cu") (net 14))
 (segment (start 89.75 68.75) (end 90.25 68.75) (width 0.5) (layer "F.Cu") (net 16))
 (segment (start 90.25 68.75) (end 90.75 68.75) (width 0.5) (layer "F.Cu") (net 16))
 (segment (start 87.76 66.76) (end 89.75 68.75) (width 0.5) (layer "F.Cu") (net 16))
 (segment (start 92.27 67.23) (end 92.72 67.23) (width 0.5) (layer "F.Cu") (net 16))
 (segment (start 87.25 66.76) (end 87.76 66.76) (width 0.5) (layer "F.Cu") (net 16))
 (segment (start 90.75 68.75) (end 92.27 67.23) (width 0.5) (layer "F.Cu") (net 16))
 (segment (start 92.72 69.77) (end 92.24 70.25) (width 0.7) (layer "F.Cu") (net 15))
 (segment (start 88.05 69.3) (end 87.25 69.3) (width 0.7) (layer "F.Cu") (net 15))
 (segment (start 87.25 69.3) (end 87.7 69.3) (width 0.7) (layer "F.Cu") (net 15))
 (segment (start 92.24 70.25) (end 89 70.25) (width 0.7) (layer "F.Cu") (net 15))
 (segment (start 89 70.25) (end 88.05 69.3) (width 0.7) (layer "F.Cu") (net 15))
 (segment (start 87.7 69.3) (end 87.75 69.25) (width 0.7) (layer "F.Cu") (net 15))
 (segment (start 87.27 64.2) (end 87.25 64.22) (width 0.7) (layer "F.Cu") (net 5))
 (segment (start 89.8 64.2) (end 87.27 64.2) (width 0.7) (layer "F.Cu") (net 5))
 (segment (start 90.25 63.75) (end 89.8 64.2) (width 0.7) (layer "F.Cu") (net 5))
 (segment (start 90.24 66.76) (end 90.25 66.75) (width 0.7) (layer "F.Cu") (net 2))
 (segment (start 112.3 64.95) (end 111.8 65.45) (width 0.5) (layer "F.Cu") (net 10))
 (segment (start 115.35 66.15) (end 114.1 67.4) (width 0.3) (layer "F.Cu") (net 10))
 (segment (start 111.8 67.2) (end 111.8 66.8) (width 0.3) (layer "F.Cu") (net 10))
 (segment (start 116.59 66.15) (end 115.35 66.15) (width 0.3) (layer "F.Cu") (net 10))
 (segment (start 113.5 64.95) (end 112.3 64.95) (width 0.5) (layer "F.Cu") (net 10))
 (segment (start 114.1 67.4) (end 112 67.4) (width 0.3) (layer "F.Cu") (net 10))
 (segment (start 112 67.4) (end 111.8 67.2) (width 0.3) (layer "F.Cu") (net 10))
 (segment (start 111.8 65.45) (end 111.8 66.8) (width 0.5) (layer "F.Cu") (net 10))
 (segment (start 115.25 65.5) (end 116.59 65.5) (width 0.3) (layer "F.Cu") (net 9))
 (segment (start 114.8 65.95) (end 115.25 65.5) (width 0.3) (layer "F.Cu") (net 9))
 (segment (start 113.5 65.95) (end 114.8 65.95) (width 0.3) (layer "F.Cu") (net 9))
 (segment (start 90.75 61.75) (end 90.25 61.75) (width 0.7) (layer "F.Cu") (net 1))
 (segment (start 91.27 61.23) (end 90.75 61.75) (width 0.7) (layer "F.Cu") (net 1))
 (segment (start 92.72 61.23) (end 91.27 61.23) (width 0.7) (layer "F.Cu") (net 1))
 (segment (start 105.25 63.35) (end 105.7 63.35) (width 0.25) (layer "F.Cu") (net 3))
 (segment (start 106.1 64.95) (end 105.25 64.1) (width 0.5) (layer "F.Cu") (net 3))
 (segment (start 104.15 63.35) (end 105.25 63.35) (width 0.5) (layer "F.Cu") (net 3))
 (segment (start 102.25 63.77) (end 103.73 63.77) (width 0.5) (layer "F.Cu") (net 3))
 (segment (start 108.225 64.95) (end 106.1 64.95) (width 0.5) (layer "F.Cu") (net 3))
 (segment (start 105.25 64.1) (end 105.25 63.35) (width 0.5) (layer "F.Cu") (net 3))
 (segment (start 103.73 63.77) (end 104.15 63.35) (width 0.5) (layer "F.Cu") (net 3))
 (segment (start 106.75 70.25) (end 102.73 70.25) (width 0.5) (layer "F.Cu") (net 8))
 (segment (start 107.5 69.5) (end 106.75 70.25) (width 0.5) (layer "F.Cu") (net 8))
 (segment (start 102.73 70.25) (end 102.25 69.77) (width 0.3) (layer "F.Cu") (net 8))
 (segment (start 108.225 63.95) (end 109.2 63.95) (width 0.5) (layer "F.Cu") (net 7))
 (segment (start 109.75 64.5) (end 109.75 69.25) (width 0.5) (layer "F.Cu") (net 7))
 (segment (start 109.75 69.25) (end 109.5 69.5) (width 0.25) (layer "F.Cu") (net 7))
 (segment (start 109.2 63.95) (end 109.75 64.5) (width 0.5) (layer "F.Cu") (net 7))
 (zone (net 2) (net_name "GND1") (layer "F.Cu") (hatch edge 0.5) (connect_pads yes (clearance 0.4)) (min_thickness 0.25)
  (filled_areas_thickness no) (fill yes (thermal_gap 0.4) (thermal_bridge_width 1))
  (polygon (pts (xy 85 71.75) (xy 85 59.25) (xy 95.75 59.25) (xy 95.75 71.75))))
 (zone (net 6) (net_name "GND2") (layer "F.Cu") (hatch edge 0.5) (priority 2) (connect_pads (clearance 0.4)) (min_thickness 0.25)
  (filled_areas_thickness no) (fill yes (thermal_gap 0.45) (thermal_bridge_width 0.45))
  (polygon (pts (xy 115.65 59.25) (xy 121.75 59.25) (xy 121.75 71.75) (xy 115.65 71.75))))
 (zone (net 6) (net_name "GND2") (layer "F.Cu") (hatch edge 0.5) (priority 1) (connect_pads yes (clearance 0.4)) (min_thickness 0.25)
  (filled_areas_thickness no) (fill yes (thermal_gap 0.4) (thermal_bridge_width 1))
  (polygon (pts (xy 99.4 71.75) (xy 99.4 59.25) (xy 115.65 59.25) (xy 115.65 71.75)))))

